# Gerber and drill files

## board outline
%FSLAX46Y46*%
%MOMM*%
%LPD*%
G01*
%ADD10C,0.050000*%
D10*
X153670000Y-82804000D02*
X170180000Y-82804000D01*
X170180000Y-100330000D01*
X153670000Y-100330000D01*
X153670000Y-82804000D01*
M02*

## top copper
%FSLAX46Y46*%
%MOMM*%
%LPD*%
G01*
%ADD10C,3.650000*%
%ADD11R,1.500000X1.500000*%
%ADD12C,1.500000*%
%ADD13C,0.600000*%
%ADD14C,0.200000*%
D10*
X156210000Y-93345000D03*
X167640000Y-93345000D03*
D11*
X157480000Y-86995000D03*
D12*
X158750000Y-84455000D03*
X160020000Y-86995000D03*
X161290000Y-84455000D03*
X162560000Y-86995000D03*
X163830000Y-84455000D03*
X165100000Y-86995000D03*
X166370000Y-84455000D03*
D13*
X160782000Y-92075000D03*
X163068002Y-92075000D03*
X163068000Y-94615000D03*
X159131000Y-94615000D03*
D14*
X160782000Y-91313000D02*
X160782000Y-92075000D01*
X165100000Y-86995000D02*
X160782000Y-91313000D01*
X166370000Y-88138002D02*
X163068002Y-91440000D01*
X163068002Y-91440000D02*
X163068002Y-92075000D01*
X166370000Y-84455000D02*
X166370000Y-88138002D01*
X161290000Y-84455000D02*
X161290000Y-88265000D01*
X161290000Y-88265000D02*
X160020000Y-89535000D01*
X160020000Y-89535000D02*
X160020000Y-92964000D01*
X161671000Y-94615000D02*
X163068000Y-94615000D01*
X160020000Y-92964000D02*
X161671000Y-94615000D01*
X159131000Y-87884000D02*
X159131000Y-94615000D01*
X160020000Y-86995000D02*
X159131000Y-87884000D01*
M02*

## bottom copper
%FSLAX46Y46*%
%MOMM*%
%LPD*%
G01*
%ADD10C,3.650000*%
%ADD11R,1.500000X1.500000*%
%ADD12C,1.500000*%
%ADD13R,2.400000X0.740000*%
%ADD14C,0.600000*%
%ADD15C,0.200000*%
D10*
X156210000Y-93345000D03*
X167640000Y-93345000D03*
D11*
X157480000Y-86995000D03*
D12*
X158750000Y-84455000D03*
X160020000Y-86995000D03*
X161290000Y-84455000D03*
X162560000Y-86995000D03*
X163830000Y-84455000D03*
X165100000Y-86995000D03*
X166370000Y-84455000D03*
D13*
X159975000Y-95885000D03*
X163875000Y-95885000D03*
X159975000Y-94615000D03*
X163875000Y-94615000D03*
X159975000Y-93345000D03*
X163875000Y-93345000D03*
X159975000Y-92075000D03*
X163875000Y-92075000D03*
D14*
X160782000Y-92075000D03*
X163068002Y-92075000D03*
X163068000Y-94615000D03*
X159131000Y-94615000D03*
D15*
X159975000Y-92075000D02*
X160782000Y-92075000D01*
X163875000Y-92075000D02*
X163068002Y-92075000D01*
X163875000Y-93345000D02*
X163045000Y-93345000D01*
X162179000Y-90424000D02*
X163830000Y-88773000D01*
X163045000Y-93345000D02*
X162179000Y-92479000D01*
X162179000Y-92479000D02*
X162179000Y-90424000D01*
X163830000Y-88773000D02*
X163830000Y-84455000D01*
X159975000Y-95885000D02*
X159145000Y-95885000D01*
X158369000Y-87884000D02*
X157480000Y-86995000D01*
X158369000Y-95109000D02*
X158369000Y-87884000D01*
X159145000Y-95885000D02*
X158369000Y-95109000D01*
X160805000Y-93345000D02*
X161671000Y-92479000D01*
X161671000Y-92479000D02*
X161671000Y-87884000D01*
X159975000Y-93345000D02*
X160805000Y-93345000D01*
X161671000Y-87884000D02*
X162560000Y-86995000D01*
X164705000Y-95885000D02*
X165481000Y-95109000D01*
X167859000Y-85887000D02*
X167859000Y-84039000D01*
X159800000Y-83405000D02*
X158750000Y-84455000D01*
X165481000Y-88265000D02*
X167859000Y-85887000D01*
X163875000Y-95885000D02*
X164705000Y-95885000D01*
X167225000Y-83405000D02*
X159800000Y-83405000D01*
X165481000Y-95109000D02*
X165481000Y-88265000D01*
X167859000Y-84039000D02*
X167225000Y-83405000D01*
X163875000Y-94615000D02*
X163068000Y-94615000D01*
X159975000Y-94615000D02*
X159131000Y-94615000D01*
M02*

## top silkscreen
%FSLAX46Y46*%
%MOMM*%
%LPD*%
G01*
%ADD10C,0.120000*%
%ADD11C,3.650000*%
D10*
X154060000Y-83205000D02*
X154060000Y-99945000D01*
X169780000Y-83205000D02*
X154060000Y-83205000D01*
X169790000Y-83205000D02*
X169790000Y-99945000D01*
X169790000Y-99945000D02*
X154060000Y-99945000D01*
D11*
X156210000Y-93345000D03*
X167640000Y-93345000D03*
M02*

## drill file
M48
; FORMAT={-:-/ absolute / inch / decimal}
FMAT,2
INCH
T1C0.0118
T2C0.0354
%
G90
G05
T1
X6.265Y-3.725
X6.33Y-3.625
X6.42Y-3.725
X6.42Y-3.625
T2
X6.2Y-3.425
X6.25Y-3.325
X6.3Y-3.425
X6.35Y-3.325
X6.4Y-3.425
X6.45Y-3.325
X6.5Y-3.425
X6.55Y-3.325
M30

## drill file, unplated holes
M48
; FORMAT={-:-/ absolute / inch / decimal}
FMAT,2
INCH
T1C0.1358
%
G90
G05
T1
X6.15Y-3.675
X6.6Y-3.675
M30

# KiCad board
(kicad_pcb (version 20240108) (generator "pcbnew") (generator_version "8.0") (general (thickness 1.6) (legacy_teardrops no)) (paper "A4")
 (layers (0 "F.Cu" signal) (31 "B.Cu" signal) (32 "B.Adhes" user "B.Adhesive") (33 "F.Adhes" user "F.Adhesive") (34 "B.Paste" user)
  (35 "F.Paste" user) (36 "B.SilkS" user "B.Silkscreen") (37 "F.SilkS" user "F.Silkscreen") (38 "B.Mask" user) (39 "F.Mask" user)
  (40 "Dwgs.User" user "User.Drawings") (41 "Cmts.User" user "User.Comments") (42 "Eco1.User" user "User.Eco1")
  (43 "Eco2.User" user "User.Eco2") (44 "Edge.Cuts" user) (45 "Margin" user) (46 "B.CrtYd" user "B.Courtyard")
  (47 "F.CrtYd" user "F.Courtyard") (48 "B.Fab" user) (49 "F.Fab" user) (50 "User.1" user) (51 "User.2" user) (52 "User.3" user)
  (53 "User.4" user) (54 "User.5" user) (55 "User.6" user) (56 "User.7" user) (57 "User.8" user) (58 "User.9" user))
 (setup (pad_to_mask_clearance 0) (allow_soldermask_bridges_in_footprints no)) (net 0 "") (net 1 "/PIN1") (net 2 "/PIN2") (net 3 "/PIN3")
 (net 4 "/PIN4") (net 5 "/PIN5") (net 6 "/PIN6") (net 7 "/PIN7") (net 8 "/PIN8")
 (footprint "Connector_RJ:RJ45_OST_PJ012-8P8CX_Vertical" (layer "F.Cu") (at 157.48 86.995)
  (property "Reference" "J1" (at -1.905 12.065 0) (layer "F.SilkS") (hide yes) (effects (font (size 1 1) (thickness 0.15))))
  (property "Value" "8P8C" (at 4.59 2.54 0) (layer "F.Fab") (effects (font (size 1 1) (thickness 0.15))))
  (fp_line (start -3.42 -3.79) (end -3.42 12.95) (stroke (width 0.12) (type solid)) (layer "F.SilkS"))
  (fp_line (start 12.3 -3.79) (end -3.42 -3.79) (stroke (width 0.12) (type solid)) (layer "F.SilkS"))
  (fp_line (start 12.31 -3.79) (end 12.31 12.95) (stroke (width 0.12) (type solid)) (layer "F.SilkS"))
  (fp_line (start 12.31 12.95) (end -3.42 12.95) (stroke (width 0.12) (type solid)) (layer "F.SilkS"))
  (pad "" np_thru_hole circle (at -1.27 6.35) (size 3.65 3.65) (drill 3.45) (layers "*.Cu" "*.SilkS" "*.Mask"))
  (pad "" np_thru_hole circle (at 10.16 6.35) (size 3.65 3.65) (drill 3.45) (layers "*.Cu" "*.SilkS" "*.Mask"))
  (pad "1" thru_hole rect (at 0 0) (size 1.5 1.5) (drill 0.9) (layers "*.Cu" "*.Mask") (remove_unused_layers no) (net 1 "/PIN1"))
  (pad "2" thru_hole circle (at 1.27 -2.54) (size 1.5 1.5) (drill 0.9) (layers "*.Cu" "*.Mask") (remove_unused_layers no) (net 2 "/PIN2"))
  (pad "3" thru_hole circle (at 2.54 0) (size 1.5 1.5) (drill 0.9) (layers "*.Cu" "*.Mask") (remove_unused_layers no) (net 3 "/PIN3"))
  (pad "4" thru_hole circle (at 3.81 -2.54) (size 1.5 1.5) (drill 0.9) (layers "*.Cu" "*.Mask") (remove_unused_layers no) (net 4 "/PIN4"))
  (pad "5" thru_hole circle (at 5.08 0) (size 1.5 1.5) (drill 0.9) (layers "*.Cu" "*.Mask") (remove_unused_layers no) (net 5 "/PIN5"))
  (pad "6" thru_hole circle (at 6.35 -2.54) (size 1.5 1.5) (drill 0.9) (layers "*.Cu" "*.Mask") (remove_unused_layers no) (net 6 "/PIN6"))
  (pad "7" thru_hole circle (at 7.62 0) (size 1.5 1.5) (drill 0.9) (layers "*.Cu" "*.Mask") (remove_unused_layers no) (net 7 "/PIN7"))
  (pad "8" thru_hole circle (at 8.89 -2.54) (size 1.5 1.5) (drill 0.9) (layers "*.Cu" "*.Mask") (remove_unused_layers no) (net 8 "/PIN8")))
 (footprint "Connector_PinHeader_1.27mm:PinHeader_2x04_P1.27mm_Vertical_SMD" (layer "B.Cu") (at 161.925 93.98)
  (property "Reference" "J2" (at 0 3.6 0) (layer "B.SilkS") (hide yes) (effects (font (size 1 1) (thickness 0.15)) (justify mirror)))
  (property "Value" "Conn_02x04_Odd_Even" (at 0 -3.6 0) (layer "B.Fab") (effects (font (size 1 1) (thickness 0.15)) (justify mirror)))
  (pad "1" smd rect (at -1.95 1.905) (size 2.4 0.74) (layers "B.Cu" "B.Paste" "B.Mask") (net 1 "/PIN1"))
  (pad "2" smd rect (at 1.95 1.905) (size 2.4 0.74) (layers "B.Cu" "B.Paste" "B.Mask") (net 2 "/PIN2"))
  (pad "3" smd rect (at -1.95 0.635) (size 2.4 0.74) (layers "B.Cu" "B.Paste" "B.Mask") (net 3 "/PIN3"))
  (pad "4" smd rect (at 1.95 0.635) (size 2.4 0.74) (layers "B.Cu" "B.Paste" "B.Mask") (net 4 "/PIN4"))
  (pad "5" smd rect (at -1.95 -0.635) (size 2.4 0.74) (layers "B.Cu" "B.Paste" "B.Mask") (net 5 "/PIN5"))
  (pad "6" smd rect (at 1.95 -0.635) (size 2.4 0.74) (layers "B.Cu" "B.Paste" "B.Mask") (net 6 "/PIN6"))
  (pad "7" smd rect (at -1.95 -1.905) (size 2.4 0.74) (layers "B.Cu" "B.Paste" "B.Mask") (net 7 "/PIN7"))
  (pad "8" smd rect (at 1.95 -1.905) (size 2.4 0.74) (layers "B.Cu" "B.Paste" "B.Mask") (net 8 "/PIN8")))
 (gr_rect (start 153.67 82.804) (end 170.18 100.33) (stroke (width 0.05) (type default)) (fill none) (layer "Edge.Cuts"))
 (segment (start 160.782 91.313) (end 160.782 92.075) (width 0.2) (layer "F.Cu") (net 7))
 (segment (start 165.1 86.995) (end 160.782 91.313) (width 0.2) (layer "F.Cu") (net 7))
 (via (at 160.782 92.075) (size 0.6) (drill 0.3) (layers "F.Cu" "B.Cu") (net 7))
 (segment (start 159.975 92.075) (end 160.782 92.075) (width 0.2) (layer "B.Cu") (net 7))
 (segment (start 166.37 88.138002) (end 163.068002 91.44) (width 0.2) (layer "F.Cu") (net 8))
 (segment (start 163.068002 91.44) (end 163.068002 92.075) (width 0.2) (layer "F.Cu") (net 8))
 (segment (start 166.37 84.455) (end 166.37 88.138002) (width 0.2) (layer "F.Cu") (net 8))
 (via (at 163.068002 92.075) (size 0.6) (drill 0.3) (layers "F.Cu" "B.Cu") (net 8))
 (segment (start 163.875 92.075) (end 163.068002 92.075) (width 0.2) (layer "B.Cu") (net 8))
 (segment (start 163.875 93.345) (end 163.045 93.345) (width 0.2) (layer "B.Cu") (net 6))
 (segment (start 162.179 90.424) (end 163.83 88.773) (width 0.2) (layer "B.Cu") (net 6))
 (segment (start 163.045 93.345) (end 162.179 92.479) (width 0.2) (layer "B.Cu") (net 6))
 (segment (start 162.179 92.479) (end 162.179 90.424) (width 0.2) (layer "B.Cu") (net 6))
 (segment (start 163.83 88.773) (end 163.83 84.455) (width 0.2) (layer "B.Cu") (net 6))
 (segment (start 159.975 95.885) (end 159.145 95.885) (width 0.2) (layer "B.Cu") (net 1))
 (segment (start 158.369 87.884) (end 157.48 86.995) (width 0.2) (layer "B.Cu") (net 1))
 (segment (start 158.369 95.109) (end 158.369 87.884) (width 0.2) (layer "B.Cu") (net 1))
 (segment (start 159.145 95.885) (end 158.369 95.109) (width 0.2) (layer "B.Cu") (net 1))
 (segment (start 160.805 93.345) (end 161.671 92.479) (width 0.2) (layer "B.Cu") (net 5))
 (segment (start 161.671 92.479) (end 161.671 87.884) (width 0.2) (layer "B.Cu") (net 5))
 (segment (start 159.975 93.345) (end 160.805 93.345) (width 0.2) (layer "B.Cu") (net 5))
 (segment (start 161.671 87.884) (end 162.56 86.995) (width 0.2) (layer "B.Cu") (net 5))
 (segment (start 164.705 95.885) (end 165.481 95.109) (width 0.2) (layer "B.Cu") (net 2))
 (segment (start 167.859 85.887) (end 167.859 84.039) (width 0.2) (layer "B.Cu") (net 2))
 (segment (start 159.8 83.405) (end 158.75 84.455) (width 0.2) (layer "B.Cu") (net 2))
 (segment (start 165.481 88.265) (end 167.859 85.887) (width 0.2) (layer "B.Cu") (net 2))
 (segment (start 163.875 95.885) (end 164.705 95.885) (width 0.2) (layer "B.Cu") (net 2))
 (segment (start 167.225 83.405) (end 159.8 83.405) (width 0.2) (layer "B.Cu") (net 2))
 (segment (start 165.481 95.109) (end 165.481 88.265) (width 0.2) (layer "B.Cu") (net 2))
 (segment (start 167.859 84.039) (end 167.225 83.405) (width 0.2) (layer "B.Cu") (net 2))
 (segment (start 161.29 84.455) (end 161.29 88.265) (width 0.2) (layer "F.Cu") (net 4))
 (segment (start 161.29 88.265) (end 160.02 89.535) (width 0.2) (layer "F.Cu") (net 4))
 (segment (start 160.02 89.535) (end 160.02 92.964) (width 0.2) (layer "F.Cu") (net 4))
 (segment (start 161.671 94.615) (end 163.068 94.615) (width 0.2) (layer "F.Cu") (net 4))
 (segment (start 160.02 92.964) (end 161.671 94.615) (width 0.2) (layer "F.Cu") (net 4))
 (via (at 163.068 94.615) (size 0.6) (drill 0.3) (layers "F.Cu" "B.Cu") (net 4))
 (segment (start 163.875 94.615) (end 163.068 94.615) (width 0.2) (layer "B.Cu") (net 4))
 (segment (start 159.131 87.884) (end 159.131 94.615) (width 0.2) (layer "F.Cu") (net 3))
 (segment (start 160.02 86.995) (end 159.131 87.884) (width 0.2) (layer "F.Cu") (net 3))
 (via (at 159.131 94.615) (size 0.6) (drill 0.3) (layers "F.Cu" "B.Cu") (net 3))
 (segment (start 159.975 94.615) (end 159.131 94.615) (width 0.2) (layer "B.Cu") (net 3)))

